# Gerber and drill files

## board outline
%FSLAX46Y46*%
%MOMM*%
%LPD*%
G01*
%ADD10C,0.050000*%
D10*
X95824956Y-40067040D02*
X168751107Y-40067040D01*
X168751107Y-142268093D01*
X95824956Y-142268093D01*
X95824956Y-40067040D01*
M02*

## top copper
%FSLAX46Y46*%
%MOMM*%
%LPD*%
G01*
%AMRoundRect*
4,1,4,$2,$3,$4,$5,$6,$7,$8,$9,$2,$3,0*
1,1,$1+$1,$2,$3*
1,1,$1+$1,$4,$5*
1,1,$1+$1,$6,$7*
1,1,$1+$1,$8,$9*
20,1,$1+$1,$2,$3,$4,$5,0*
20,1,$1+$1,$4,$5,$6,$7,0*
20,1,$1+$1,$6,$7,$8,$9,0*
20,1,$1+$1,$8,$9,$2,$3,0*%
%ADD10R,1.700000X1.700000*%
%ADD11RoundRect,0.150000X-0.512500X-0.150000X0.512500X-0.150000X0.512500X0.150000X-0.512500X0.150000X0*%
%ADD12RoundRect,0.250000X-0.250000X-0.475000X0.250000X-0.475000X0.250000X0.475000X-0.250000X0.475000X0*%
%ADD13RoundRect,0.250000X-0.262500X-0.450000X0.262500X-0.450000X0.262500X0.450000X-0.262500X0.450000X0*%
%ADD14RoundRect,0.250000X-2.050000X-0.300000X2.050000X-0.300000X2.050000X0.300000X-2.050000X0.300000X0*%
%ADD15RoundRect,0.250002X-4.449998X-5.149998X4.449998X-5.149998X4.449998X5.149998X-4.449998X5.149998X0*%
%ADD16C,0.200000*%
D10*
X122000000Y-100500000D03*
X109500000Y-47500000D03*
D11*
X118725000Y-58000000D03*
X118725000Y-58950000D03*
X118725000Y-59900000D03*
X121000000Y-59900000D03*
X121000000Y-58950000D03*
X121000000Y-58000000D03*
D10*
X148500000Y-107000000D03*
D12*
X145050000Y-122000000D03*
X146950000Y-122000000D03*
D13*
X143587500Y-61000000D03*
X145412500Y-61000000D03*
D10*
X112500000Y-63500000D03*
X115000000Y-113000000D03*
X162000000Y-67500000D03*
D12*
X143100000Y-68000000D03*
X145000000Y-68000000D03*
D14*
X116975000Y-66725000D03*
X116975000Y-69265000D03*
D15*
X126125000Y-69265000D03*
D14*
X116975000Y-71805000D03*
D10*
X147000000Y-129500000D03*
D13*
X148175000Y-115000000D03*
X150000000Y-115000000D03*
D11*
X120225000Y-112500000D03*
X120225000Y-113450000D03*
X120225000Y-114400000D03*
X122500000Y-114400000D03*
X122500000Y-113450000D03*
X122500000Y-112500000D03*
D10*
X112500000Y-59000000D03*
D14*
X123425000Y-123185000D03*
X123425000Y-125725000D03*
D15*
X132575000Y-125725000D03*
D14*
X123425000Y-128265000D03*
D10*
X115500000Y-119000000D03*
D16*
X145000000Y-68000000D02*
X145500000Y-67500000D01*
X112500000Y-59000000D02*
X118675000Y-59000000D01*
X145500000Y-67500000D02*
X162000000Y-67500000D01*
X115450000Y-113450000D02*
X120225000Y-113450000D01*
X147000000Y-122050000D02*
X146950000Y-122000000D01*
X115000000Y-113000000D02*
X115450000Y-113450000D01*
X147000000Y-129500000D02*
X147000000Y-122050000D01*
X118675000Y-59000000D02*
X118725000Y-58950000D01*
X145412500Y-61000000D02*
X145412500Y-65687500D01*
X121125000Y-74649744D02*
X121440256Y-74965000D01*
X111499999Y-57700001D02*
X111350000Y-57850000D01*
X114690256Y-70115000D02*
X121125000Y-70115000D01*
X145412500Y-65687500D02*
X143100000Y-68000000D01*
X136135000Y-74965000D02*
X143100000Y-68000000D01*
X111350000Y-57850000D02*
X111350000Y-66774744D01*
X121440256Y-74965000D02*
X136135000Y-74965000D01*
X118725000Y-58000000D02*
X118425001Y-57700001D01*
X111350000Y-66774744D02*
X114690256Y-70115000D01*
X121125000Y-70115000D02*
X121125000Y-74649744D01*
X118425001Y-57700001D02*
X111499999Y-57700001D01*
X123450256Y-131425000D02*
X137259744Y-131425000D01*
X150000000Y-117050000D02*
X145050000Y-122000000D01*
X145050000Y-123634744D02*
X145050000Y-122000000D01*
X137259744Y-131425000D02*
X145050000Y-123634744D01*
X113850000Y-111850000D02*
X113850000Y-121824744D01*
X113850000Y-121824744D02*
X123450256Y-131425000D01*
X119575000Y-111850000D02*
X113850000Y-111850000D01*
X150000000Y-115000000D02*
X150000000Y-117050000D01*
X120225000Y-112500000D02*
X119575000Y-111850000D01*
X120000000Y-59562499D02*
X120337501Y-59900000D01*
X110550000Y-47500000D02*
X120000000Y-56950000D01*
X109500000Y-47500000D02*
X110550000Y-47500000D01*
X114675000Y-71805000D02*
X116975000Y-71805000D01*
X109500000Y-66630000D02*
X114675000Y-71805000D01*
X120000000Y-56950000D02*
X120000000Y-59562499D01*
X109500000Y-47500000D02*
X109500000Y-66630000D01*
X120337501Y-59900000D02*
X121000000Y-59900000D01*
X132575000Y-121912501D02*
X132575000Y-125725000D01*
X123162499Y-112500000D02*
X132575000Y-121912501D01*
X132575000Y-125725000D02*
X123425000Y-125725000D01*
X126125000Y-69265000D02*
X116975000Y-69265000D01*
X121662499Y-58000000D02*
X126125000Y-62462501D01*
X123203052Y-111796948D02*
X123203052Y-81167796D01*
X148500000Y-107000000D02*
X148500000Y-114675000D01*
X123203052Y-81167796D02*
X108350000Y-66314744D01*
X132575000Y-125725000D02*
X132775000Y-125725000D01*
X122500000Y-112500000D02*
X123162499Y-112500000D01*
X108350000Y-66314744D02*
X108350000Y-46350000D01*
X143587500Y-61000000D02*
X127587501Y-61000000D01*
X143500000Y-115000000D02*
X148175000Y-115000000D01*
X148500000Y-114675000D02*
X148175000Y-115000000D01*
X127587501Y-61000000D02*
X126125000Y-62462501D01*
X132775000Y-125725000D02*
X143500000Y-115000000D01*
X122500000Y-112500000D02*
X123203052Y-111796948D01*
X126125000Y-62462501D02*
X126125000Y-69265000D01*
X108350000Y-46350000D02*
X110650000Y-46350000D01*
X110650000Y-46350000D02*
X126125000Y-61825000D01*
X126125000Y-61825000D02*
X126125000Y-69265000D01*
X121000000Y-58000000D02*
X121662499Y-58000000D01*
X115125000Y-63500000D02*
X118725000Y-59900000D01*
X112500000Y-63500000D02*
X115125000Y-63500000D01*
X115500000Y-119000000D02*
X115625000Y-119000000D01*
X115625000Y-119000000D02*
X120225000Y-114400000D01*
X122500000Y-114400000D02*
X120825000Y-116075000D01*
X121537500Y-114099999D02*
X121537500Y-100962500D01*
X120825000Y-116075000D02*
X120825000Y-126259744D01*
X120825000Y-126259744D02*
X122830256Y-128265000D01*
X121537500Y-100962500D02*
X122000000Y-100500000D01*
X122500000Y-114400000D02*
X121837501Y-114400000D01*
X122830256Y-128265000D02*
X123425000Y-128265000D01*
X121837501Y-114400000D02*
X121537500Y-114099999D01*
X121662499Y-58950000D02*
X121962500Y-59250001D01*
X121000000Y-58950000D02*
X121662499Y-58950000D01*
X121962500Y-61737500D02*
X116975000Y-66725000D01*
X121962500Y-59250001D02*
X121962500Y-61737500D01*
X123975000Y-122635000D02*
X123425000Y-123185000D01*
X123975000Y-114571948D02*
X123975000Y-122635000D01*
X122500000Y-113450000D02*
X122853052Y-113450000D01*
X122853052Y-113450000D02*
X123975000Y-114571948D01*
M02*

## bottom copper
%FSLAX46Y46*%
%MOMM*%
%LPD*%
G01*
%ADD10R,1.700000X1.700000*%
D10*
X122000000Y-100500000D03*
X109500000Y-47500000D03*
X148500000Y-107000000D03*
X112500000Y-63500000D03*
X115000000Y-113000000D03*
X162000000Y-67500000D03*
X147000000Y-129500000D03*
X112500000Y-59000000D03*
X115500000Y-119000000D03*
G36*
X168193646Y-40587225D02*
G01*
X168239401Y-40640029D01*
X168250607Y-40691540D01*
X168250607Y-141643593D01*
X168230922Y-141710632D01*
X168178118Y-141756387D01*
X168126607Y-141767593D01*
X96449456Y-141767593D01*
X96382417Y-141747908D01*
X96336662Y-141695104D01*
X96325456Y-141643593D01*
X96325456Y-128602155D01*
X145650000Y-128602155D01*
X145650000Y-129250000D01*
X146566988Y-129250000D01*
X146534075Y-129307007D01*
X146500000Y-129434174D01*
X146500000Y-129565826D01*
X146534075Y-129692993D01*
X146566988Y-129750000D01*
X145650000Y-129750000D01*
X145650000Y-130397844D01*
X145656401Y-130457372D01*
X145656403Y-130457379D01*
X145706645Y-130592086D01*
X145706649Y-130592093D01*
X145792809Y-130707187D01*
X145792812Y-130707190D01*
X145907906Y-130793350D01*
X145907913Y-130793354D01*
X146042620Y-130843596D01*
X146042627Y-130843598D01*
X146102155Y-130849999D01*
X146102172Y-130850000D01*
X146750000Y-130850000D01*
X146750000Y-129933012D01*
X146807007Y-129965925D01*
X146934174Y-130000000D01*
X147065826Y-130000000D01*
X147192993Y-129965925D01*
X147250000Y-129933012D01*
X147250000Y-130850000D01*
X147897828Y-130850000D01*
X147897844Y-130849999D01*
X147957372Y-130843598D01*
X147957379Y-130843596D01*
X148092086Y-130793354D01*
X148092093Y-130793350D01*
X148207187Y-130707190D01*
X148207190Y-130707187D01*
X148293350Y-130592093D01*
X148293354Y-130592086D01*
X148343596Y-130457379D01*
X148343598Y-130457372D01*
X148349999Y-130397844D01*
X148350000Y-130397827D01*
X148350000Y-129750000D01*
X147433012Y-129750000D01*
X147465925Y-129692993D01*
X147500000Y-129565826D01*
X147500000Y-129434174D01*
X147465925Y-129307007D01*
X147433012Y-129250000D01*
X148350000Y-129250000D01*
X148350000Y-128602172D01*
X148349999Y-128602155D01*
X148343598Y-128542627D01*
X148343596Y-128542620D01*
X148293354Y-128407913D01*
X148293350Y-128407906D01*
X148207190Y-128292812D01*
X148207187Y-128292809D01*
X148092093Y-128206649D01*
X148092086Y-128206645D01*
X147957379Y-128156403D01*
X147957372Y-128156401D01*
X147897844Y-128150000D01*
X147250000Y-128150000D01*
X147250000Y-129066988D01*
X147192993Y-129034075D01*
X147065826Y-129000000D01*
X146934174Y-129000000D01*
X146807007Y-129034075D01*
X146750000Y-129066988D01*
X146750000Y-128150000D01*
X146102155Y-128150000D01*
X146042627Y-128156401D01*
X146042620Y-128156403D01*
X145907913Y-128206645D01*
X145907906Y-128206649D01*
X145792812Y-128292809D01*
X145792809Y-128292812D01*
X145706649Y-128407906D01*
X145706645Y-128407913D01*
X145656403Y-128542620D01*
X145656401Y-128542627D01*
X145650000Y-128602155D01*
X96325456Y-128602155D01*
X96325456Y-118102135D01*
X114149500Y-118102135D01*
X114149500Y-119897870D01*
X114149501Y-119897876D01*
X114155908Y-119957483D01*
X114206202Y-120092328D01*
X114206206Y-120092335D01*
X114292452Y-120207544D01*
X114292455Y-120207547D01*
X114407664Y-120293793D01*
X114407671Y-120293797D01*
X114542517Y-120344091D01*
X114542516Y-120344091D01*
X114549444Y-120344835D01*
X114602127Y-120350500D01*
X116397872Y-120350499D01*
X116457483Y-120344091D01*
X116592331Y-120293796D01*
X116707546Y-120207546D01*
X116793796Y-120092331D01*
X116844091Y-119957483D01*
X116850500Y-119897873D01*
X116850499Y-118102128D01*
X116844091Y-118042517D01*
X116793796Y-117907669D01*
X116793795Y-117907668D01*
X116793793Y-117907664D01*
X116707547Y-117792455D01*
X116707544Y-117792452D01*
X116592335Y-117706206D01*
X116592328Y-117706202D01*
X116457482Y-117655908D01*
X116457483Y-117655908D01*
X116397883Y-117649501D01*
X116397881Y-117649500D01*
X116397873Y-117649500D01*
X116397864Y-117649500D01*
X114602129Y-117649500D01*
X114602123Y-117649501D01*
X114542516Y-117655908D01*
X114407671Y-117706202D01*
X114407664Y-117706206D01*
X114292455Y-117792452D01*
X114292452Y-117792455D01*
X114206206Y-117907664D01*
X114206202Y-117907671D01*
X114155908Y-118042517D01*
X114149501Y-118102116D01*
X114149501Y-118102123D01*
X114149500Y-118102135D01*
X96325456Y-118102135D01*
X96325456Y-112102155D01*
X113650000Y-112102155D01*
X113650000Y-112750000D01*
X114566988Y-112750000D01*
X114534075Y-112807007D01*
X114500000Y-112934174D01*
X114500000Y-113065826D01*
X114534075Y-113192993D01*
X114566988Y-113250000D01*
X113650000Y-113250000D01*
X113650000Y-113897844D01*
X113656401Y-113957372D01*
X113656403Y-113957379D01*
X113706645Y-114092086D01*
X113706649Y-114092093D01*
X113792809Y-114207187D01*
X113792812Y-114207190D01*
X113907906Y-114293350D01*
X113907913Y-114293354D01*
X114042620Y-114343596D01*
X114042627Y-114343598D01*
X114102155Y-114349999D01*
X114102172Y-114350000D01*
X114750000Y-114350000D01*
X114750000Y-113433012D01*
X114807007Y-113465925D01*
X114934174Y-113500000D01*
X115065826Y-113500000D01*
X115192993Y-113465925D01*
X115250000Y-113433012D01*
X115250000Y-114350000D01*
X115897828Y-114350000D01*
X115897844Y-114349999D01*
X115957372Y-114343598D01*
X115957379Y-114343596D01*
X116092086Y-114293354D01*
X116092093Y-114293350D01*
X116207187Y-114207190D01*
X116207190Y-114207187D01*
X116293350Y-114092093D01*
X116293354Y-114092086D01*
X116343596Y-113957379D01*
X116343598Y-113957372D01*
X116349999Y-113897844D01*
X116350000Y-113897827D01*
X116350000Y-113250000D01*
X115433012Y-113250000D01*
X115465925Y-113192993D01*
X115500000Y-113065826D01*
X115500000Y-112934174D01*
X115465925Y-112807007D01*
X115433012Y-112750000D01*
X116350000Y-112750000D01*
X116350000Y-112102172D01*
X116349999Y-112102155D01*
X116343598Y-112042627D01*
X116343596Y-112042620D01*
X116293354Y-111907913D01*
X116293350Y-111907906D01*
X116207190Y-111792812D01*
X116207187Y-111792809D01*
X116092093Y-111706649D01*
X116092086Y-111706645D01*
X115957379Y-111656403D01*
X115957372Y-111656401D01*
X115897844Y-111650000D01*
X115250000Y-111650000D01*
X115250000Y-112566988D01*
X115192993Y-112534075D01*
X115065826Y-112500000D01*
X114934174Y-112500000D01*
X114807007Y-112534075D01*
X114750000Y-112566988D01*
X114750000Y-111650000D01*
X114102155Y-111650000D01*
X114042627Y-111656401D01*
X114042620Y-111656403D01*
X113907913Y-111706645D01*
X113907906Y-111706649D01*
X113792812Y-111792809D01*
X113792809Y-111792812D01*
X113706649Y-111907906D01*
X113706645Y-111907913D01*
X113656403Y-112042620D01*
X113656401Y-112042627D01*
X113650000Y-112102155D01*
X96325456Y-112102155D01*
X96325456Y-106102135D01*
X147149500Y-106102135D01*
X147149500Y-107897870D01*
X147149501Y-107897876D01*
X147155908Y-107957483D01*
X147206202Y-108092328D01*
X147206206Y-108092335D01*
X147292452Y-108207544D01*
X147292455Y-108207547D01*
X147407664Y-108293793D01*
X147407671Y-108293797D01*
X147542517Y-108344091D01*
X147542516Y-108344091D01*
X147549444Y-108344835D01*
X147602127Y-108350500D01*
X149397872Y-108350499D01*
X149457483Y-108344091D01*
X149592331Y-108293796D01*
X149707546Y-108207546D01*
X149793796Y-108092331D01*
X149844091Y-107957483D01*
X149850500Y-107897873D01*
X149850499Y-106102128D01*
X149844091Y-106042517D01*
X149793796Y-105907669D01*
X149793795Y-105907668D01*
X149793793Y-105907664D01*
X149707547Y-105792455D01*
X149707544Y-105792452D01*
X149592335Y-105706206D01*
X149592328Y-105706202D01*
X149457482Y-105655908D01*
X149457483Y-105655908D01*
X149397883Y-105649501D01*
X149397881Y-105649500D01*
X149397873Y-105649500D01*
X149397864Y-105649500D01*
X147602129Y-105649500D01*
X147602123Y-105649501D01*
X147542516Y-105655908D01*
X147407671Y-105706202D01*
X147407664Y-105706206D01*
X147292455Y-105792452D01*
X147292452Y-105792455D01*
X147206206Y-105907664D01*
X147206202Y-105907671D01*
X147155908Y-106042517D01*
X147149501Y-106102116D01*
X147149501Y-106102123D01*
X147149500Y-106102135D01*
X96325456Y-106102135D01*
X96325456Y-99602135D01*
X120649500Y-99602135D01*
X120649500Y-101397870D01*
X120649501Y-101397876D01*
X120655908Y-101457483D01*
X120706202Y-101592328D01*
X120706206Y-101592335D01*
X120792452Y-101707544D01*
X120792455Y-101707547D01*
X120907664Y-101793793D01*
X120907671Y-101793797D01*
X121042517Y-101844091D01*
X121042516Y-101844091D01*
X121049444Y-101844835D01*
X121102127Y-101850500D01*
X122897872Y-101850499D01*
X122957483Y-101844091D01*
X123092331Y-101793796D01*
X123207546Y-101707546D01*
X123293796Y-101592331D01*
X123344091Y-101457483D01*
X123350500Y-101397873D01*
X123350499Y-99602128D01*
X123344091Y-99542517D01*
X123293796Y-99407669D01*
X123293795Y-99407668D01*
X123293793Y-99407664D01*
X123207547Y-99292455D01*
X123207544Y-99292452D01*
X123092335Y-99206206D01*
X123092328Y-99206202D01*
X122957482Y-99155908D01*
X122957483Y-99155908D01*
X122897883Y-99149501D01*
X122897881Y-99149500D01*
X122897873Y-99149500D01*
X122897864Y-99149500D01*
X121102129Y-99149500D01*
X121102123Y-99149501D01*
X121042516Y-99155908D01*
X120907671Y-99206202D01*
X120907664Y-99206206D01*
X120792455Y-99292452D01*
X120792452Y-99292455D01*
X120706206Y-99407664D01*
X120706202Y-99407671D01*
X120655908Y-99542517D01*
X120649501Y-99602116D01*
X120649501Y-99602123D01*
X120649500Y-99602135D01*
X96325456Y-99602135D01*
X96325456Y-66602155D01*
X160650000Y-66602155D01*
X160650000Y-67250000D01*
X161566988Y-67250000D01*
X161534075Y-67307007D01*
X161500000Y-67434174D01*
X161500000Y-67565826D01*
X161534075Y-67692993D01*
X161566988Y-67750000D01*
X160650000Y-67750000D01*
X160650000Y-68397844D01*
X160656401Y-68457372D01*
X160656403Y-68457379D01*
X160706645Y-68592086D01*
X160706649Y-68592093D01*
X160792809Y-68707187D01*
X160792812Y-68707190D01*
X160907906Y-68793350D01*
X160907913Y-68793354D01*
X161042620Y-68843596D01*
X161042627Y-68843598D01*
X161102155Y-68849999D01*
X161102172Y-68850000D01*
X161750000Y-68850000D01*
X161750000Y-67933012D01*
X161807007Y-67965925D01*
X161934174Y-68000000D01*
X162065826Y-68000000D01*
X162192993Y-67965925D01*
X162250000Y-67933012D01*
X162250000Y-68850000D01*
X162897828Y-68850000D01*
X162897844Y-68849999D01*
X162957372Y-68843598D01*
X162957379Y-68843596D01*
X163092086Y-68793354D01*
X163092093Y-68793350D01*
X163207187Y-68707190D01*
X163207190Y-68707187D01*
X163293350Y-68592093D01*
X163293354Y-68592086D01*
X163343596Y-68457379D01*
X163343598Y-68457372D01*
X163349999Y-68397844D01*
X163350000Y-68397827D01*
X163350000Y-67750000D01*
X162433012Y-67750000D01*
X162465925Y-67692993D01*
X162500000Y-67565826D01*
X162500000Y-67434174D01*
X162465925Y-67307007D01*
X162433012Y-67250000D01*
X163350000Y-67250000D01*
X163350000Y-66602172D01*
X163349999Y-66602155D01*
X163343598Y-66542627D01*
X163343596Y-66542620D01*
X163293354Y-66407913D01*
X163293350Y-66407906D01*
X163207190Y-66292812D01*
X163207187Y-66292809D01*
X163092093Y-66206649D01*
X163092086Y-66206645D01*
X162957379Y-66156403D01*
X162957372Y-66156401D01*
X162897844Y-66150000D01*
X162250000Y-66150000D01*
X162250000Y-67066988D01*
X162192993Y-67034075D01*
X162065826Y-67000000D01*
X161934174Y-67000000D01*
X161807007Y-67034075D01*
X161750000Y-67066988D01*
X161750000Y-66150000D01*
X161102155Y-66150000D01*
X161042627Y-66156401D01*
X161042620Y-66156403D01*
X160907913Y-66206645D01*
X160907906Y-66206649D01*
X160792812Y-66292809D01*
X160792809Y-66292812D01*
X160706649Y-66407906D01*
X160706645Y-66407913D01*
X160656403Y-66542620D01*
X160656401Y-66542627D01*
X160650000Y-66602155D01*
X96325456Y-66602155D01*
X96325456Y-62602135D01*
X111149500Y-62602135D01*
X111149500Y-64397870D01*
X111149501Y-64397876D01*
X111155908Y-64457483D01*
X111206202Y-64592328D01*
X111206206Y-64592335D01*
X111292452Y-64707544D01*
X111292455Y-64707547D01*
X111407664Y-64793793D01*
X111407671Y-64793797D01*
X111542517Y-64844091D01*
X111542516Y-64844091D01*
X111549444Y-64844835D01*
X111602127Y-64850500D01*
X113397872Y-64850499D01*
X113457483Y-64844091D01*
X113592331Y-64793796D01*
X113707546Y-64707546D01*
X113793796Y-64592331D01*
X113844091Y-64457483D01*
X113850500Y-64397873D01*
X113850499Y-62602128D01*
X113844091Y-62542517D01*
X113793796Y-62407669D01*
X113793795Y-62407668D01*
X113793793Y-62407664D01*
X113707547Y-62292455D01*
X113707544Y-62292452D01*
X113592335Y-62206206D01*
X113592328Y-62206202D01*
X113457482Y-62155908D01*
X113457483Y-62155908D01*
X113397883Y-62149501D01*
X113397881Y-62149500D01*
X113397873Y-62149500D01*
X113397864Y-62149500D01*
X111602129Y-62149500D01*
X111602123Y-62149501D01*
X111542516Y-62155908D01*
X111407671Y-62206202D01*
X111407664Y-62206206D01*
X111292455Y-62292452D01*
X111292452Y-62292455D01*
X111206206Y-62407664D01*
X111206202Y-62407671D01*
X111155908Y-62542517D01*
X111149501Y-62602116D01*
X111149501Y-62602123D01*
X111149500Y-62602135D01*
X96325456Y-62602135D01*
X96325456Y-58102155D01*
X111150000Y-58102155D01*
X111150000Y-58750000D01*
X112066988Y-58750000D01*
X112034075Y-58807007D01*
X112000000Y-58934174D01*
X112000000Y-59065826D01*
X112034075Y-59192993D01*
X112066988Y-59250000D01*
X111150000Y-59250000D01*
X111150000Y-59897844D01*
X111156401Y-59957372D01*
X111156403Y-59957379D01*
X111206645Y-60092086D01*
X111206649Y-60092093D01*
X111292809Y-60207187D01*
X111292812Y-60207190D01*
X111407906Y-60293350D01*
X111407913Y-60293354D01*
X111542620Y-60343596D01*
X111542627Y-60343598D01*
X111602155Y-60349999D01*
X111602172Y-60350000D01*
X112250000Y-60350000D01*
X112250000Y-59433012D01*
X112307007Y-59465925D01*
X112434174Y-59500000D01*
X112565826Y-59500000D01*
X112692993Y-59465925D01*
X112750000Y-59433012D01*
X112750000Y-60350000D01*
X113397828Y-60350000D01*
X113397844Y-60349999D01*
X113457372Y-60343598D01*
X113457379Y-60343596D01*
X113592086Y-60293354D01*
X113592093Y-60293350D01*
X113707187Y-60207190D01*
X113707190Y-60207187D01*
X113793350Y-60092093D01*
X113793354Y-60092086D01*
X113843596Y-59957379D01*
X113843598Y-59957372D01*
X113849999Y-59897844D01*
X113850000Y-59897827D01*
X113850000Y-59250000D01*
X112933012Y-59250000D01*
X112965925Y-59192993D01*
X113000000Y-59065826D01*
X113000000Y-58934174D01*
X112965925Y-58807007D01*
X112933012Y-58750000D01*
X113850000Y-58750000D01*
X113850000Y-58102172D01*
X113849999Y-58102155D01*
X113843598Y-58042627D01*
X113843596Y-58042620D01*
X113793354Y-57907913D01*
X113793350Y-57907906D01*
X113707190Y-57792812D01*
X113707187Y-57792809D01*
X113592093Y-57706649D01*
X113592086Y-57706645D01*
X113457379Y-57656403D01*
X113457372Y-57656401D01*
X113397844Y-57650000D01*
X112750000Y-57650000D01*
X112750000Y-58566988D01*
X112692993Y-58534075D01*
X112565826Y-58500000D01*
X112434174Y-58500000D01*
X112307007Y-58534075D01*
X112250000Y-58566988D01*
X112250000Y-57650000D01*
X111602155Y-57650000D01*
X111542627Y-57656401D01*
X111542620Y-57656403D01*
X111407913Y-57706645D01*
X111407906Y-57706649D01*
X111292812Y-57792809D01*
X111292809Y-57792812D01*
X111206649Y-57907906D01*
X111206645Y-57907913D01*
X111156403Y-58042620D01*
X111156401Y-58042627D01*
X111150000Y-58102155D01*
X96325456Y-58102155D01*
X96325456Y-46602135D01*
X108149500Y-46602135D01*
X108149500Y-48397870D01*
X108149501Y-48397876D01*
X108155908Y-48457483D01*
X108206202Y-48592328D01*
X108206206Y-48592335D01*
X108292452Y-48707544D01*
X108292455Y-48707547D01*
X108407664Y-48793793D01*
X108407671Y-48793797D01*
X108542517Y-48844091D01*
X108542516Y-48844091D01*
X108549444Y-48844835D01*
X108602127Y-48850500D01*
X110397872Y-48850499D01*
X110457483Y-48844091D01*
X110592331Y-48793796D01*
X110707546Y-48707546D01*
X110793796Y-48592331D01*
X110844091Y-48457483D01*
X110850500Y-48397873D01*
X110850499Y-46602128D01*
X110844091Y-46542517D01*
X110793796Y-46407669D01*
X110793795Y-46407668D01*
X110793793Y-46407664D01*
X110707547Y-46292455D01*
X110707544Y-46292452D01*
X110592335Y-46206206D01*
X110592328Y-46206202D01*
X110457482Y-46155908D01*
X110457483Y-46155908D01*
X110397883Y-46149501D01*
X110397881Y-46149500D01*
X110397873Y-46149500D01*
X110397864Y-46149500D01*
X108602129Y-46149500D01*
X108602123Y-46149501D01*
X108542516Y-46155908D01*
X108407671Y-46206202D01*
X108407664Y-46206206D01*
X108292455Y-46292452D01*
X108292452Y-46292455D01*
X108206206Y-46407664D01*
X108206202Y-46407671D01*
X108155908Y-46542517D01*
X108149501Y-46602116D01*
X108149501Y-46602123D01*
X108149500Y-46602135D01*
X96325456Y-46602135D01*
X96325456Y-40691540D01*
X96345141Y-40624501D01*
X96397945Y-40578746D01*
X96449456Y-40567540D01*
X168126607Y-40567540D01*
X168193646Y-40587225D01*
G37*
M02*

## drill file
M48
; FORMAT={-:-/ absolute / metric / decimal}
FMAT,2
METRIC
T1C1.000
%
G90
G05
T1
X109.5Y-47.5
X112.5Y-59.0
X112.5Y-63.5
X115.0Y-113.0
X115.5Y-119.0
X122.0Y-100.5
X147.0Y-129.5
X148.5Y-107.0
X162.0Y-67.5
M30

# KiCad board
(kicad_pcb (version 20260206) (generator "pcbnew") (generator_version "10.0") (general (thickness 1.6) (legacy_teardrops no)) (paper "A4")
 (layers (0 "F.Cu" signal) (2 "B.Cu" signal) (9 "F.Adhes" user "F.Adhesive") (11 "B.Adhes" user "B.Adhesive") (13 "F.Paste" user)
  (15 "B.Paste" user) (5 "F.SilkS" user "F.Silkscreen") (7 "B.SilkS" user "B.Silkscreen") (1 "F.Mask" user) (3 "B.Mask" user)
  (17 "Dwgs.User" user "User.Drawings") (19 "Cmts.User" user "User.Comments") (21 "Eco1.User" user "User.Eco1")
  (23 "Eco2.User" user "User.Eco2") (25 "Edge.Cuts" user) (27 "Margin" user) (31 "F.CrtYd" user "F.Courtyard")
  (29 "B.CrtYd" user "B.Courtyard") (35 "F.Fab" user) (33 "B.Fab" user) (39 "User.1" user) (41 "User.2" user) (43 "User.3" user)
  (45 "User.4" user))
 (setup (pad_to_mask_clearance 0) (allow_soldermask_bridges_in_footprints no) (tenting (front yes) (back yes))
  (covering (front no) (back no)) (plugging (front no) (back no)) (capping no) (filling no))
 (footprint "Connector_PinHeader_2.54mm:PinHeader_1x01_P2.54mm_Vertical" (layer "F.Cu") (at 122 100.5)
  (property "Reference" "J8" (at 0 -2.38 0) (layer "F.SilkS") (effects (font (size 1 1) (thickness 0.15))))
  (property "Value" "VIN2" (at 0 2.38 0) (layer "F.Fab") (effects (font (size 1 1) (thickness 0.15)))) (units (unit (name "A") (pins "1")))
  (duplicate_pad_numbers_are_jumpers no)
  (pad "1" thru_hole rect (at 0 0) (size 1.7 1.7) (drill 1) (layers "*.Cu" "*.Mask") (remove_unused_layers no) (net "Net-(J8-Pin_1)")))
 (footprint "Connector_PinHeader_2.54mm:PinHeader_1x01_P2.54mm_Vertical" (layer "F.Cu") (at 109.5 47.5)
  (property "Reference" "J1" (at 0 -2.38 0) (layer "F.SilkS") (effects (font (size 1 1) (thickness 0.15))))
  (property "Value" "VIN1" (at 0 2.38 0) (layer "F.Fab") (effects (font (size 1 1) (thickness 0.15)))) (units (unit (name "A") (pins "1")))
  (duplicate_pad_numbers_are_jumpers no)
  (pad "1" thru_hole rect (at 0 0) (size 1.7 1.7) (drill 1) (layers "*.Cu" "*.Mask") (remove_unused_layers no) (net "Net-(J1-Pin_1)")))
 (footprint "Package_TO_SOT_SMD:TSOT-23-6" (layer "F.Cu") (at 119.8625 58.95)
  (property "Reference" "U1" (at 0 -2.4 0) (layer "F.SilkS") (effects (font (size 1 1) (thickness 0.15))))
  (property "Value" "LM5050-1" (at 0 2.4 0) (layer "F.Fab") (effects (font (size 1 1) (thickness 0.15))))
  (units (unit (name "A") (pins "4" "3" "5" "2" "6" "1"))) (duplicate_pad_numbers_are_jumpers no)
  (pad "1" smd roundrect (at -1.1375 -0.95) (size 1.325 0.6) (layers "F.Cu" "F.Mask" "F.Paste") (roundrect_rratio 0.25) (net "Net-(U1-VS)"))
  (pad "2" smd roundrect (at -1.1375 0) (size 1.325 0.6) (layers "F.Cu" "F.Mask" "F.Paste") (roundrect_rratio 0.25) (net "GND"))
  (pad "3" smd roundrect (at -1.1375 0.95) (size 1.325 0.6) (layers "F.Cu" "F.Mask" "F.Paste") (roundrect_rratio 0.25)
   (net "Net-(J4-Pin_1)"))
  (pad "4" smd roundrect (at 1.1375 0.95) (size 1.325 0.6) (layers "F.Cu" "F.Mask" "F.Paste") (roundrect_rratio 0.25) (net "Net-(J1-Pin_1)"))
  (pad "5" smd roundrect (at 1.1375 0) (size 1.325 0.6) (layers "F.Cu" "F.Mask" "F.Paste") (roundrect_rratio 0.25) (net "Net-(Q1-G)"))
  (pad "6" smd roundrect (at 1.1375 -0.95) (size 1.325 0.6) (layers "F.Cu" "F.Mask" "F.Paste") (roundrect_rratio 0.25)
   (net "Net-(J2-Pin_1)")))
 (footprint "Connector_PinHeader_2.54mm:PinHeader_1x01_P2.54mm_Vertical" (layer "F.Cu") (at 148.5 107)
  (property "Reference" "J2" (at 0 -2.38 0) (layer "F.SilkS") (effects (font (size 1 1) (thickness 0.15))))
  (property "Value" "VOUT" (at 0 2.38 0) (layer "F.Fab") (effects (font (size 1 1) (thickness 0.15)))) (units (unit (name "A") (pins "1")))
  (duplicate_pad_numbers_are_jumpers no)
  (pad "1" thru_hole rect (at 0 0) (size 1.7 1.7) (drill 1) (layers "*.Cu" "*.Mask") (remove_unused_layers no) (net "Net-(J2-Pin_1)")))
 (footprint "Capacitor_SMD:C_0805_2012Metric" (layer "F.Cu") (at 146 122)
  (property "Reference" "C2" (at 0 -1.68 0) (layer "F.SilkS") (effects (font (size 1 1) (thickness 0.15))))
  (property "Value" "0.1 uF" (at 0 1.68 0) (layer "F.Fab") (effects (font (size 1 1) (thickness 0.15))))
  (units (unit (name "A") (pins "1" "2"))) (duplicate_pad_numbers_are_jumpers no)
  (pad "1" smd roundrect (at -0.95 0) (size 1 1.45) (layers "F.Cu" "F.Mask" "F.Paste") (roundrect_rratio 0.25) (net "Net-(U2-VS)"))
  (pad "2" smd roundrect (at 0.95 0) (size 1 1.45) (layers "F.Cu" "F.Mask" "F.Paste") (roundrect_rratio 0.25) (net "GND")))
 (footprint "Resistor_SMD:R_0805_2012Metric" (layer "F.Cu") (at 144.5 61)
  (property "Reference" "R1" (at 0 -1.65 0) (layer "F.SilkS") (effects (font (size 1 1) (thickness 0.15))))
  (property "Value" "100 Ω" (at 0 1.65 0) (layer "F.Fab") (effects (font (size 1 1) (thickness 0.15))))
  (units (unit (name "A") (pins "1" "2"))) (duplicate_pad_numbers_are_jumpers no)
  (pad "1" smd roundrect (at -0.9125 0) (size 1.025 1.4) (layers "F.Cu" "F.Mask" "F.Paste") (roundrect_rratio 0.243902)
   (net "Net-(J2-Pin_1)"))
  (pad "2" smd roundrect (at 0.9125 0) (size 1.025 1.4) (layers "F.Cu" "F.Mask" "F.Paste") (roundrect_rratio 0.243902) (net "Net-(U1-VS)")))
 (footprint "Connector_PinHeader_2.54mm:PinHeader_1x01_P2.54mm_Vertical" (layer "F.Cu") (at 112.5 63.5)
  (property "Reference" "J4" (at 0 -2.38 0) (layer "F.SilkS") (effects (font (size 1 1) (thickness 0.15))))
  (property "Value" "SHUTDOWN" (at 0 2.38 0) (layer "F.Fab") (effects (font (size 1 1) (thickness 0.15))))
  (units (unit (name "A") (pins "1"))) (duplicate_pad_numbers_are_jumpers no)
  (pad "1" thru_hole rect (at 0 0) (size 1.7 1.7) (drill 1) (layers "*.Cu" "*.Mask") (remove_unused_layers no) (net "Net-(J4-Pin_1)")))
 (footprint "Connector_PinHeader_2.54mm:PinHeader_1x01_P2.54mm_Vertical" (layer "F.Cu") (at 115 113)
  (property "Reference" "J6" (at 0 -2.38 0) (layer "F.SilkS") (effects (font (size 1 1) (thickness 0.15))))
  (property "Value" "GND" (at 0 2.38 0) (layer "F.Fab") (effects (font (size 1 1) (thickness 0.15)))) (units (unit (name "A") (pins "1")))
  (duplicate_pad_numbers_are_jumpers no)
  (pad "1" thru_hole rect (at 0 0) (size 1.7 1.7) (drill 1) (layers "*.Cu" "*.Mask") (remove_unused_layers no) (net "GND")))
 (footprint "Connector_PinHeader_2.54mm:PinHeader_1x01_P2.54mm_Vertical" (layer "F.Cu") (at 162 67.5)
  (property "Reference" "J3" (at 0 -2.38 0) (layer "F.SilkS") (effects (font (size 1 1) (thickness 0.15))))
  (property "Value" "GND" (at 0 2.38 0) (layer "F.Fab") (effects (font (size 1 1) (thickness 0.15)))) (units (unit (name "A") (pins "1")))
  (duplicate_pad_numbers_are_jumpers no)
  (pad "1" thru_hole rect (at 0 0) (size 1.7 1.7) (drill 1) (layers "*.Cu" "*.Mask") (remove_unused_layers no) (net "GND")))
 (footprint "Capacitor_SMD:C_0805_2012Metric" (layer "F.Cu") (at 144.05 68)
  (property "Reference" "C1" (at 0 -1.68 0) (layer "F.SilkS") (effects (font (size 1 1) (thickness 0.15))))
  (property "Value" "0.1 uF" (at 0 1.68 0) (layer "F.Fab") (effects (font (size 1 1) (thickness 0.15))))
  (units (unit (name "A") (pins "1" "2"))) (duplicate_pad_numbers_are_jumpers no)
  (pad "1" smd roundrect (at -0.95 0) (size 1 1.45) (layers "F.Cu" "F.Mask" "F.Paste") (roundrect_rratio 0.25) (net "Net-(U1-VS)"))
  (pad "2" smd roundrect (at 0.95 0) (size 1 1.45) (layers "F.Cu" "F.Mask" "F.Paste") (roundrect_rratio 0.25) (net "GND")))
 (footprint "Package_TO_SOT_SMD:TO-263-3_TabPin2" (layer "F.Cu") (at 124.625 69.265)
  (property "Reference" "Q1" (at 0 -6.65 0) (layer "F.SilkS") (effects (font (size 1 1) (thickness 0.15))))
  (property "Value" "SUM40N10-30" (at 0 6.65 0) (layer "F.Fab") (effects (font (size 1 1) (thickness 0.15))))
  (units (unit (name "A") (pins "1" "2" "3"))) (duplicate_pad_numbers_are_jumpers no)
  (pad "" smd roundrect (at -0.925 -2.775) (size 4.55 5.25) (layers "F.Paste") (roundrect_rratio 0.054945))
  (pad "" smd roundrect (at -0.925 2.775) (size 4.55 5.25) (layers "F.Paste") (roundrect_rratio 0.054945))
  (pad "" smd roundrect (at 3.925 -2.775) (size 4.55 5.25) (layers "F.Paste") (roundrect_rratio 0.054945))
  (pad "" smd roundrect (at 3.925 2.775) (size 4.55 5.25) (layers "F.Paste") (roundrect_rratio 0.054945))
  (pad "1" smd roundrect (at -7.65 -2.54) (size 4.6 1.1) (layers "F.Cu" "F.Mask" "F.Paste") (roundrect_rratio 0.227273) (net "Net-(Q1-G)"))
  (pad "2" smd roundrect (at -7.65 0) (size 4.6 1.1) (layers "F.Cu" "F.Mask" "F.Paste") (roundrect_rratio 0.227273) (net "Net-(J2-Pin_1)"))
  (pad "2" smd roundrect (at 1.5 0) (size 9.4 10.8) (layers "F.Cu" "F.Mask") (roundrect_rratio 0.026596) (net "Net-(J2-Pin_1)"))
  (pad "3" smd roundrect (at -7.65 2.54) (size 4.6 1.1) (layers "F.Cu" "F.Mask" "F.Paste") (roundrect_rratio 0.227273)
   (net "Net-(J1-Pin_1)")))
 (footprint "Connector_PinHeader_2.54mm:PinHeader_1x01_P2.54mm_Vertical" (layer "F.Cu") (at 147 129.5)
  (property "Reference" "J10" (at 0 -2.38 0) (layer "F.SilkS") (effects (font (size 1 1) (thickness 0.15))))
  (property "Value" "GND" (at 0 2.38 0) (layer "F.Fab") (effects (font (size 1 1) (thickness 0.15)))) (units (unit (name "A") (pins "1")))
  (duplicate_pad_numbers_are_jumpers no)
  (pad "1" thru_hole rect (at 0 0) (size 1.7 1.7) (drill 1) (layers "*.Cu" "*.Mask") (remove_unused_layers no) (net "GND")))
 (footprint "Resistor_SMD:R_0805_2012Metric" (layer "F.Cu") (at 149.0875 115)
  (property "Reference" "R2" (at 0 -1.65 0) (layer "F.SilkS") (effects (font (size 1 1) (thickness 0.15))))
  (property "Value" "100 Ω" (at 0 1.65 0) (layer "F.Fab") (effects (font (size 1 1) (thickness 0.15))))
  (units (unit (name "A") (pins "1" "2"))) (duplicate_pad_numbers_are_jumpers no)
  (pad "1" smd roundrect (at -0.9125 0) (size 1.025 1.4) (layers "F.Cu" "F.Mask" "F.Paste") (roundrect_rratio 0.243902)
   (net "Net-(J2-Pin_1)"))
  (pad "2" smd roundrect (at 0.9125 0) (size 1.025 1.4) (layers "F.Cu" "F.Mask" "F.Paste") (roundrect_rratio 0.243902) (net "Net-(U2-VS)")))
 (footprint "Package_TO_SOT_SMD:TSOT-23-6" (layer "F.Cu") (at 121.3625 113.45)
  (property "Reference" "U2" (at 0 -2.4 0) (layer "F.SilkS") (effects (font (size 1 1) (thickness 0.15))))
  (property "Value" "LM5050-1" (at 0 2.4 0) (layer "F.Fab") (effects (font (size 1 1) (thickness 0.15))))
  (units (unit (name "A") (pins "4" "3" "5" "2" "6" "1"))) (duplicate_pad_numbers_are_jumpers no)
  (pad "1" smd roundrect (at -1.1375 -0.95) (size 1.325 0.6) (layers "F.Cu" "F.Mask" "F.Paste") (roundrect_rratio 0.25) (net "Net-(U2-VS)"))
  (pad "2" smd roundrect (at -1.1375 0) (size 1.325 0.6) (layers "F.Cu" "F.Mask" "F.Paste") (roundrect_rratio 0.25) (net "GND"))
  (pad "3" smd roundrect (at -1.1375 0.95) (size 1.325 0.6) (layers "F.Cu" "F.Mask" "F.Paste") (roundrect_rratio 0.25)
   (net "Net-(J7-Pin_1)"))
  (pad "4" smd roundrect (at 1.1375 0.95) (size 1.325 0.6) (layers "F.Cu" "F.Mask" "F.Paste") (roundrect_rratio 0.25) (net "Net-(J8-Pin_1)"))
  (pad "5" smd roundrect (at 1.1375 0) (size 1.325 0.6) (layers "F.Cu" "F.Mask" "F.Paste") (roundrect_rratio 0.25) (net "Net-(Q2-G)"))
  (pad "6" smd roundrect (at 1.1375 -0.95) (size 1.325 0.6) (layers "F.Cu" "F.Mask" "F.Paste") (roundrect_rratio 0.25)
   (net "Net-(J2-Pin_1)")))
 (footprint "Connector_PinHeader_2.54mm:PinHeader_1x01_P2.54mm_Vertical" (layer "F.Cu") (at 112.5 59)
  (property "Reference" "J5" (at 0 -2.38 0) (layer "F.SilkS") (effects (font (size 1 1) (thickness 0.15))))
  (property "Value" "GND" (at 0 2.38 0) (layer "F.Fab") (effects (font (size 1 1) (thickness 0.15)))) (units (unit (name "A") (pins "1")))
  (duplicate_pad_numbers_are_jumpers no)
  (pad "1" thru_hole rect (at 0 0) (size 1.7 1.7) (drill 1) (layers "*.Cu" "*.Mask") (remove_unused_layers no) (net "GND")))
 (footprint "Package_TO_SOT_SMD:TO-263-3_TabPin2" (layer "F.Cu") (at 131.075 125.725)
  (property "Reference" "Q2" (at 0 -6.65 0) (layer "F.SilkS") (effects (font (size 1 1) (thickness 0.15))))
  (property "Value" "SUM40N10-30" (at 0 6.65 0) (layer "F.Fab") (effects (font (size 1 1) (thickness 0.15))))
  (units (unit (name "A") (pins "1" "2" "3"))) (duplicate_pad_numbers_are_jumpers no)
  (pad "" smd roundrect (at -0.925 -2.775) (size 4.55 5.25) (layers "F.Paste") (roundrect_rratio 0.054945))
  (pad "" smd roundrect (at -0.925 2.775) (size 4.55 5.25) (layers "F.Paste") (roundrect_rratio 0.054945))
  (pad "" smd roundrect (at 3.925 -2.775) (size 4.55 5.25) (layers "F.Paste") (roundrect_rratio 0.054945))
  (pad "" smd roundrect (at 3.925 2.775) (size 4.55 5.25) (layers "F.Paste") (roundrect_rratio 0.054945))
  (pad "1" smd roundrect (at -7.65 -2.54) (size 4.6 1.1) (layers "F.Cu" "F.Mask" "F.Paste") (roundrect_rratio 0.227273) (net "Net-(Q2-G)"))
  (pad "2" smd roundrect (at -7.65 0) (size 4.6 1.1) (layers "F.Cu" "F.Mask" "F.Paste") (roundrect_rratio 0.227273) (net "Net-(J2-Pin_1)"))
  (pad "2" smd roundrect (at 1.5 0) (size 9.4 10.8) (layers "F.Cu" "F.Mask") (roundrect_rratio 0.026596) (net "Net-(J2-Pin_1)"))
  (pad "3" smd roundrect (at -7.65 2.54) (size 4.6 1.1) (layers "F.Cu" "F.Mask" "F.Paste") (roundrect_rratio 0.227273)
   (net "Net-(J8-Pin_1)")))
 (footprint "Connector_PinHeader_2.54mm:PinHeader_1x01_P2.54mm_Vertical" (layer "F.Cu") (at 115.5 119)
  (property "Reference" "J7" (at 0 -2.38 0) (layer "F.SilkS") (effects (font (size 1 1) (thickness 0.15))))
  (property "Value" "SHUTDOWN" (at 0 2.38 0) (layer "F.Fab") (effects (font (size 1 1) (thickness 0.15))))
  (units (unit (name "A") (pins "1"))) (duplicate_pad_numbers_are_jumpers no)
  (pad "1" thru_hole rect (at 0 0) (size 1.7 1.7) (drill 1) (layers "*.Cu" "*.Mask") (remove_unused_layers no) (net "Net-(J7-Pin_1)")))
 (gr_rect (start 95.824956 40.06704) (end 168.751107 142.268093) (stroke (width 0.05) (type default)) (fill no) (layer "Edge.Cuts"))
 (segment (start 145 68) (end 145.5 67.5) (width 0.2) (layer "F.Cu") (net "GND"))
 (segment (start 112.5 59) (end 118.675 59) (width 0.2) (layer "F.Cu") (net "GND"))
 (segment (start 145.5 67.5) (end 162 67.5) (width 0.2) (layer "F.Cu") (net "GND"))
 (segment (start 115.45 113.45) (end 120.225 113.45) (width 0.2) (layer "F.Cu") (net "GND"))
 (segment (start 147 122.05) (end 146.95 122) (width 0.2) (layer "F.Cu") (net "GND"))
 (segment (start 115 113) (end 115.45 113.45) (width 0.2) (layer "F.Cu") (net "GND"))
 (segment (start 147 129.5) (end 147 122.05) (width 0.2) (layer "F.Cu") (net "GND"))
 (segment (start 118.675 59) (end 118.725 58.95) (width 0.2) (layer "F.Cu") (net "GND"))
 (segment (start 145.4125 61) (end 145.4125 65.6875) (width 0.2) (layer "F.Cu") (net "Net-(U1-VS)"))
 (segment (start 121.125 74.649744) (end 121.440256 74.965) (width 0.2) (layer "F.Cu") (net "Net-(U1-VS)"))
 (segment (start 111.499999 57.700001) (end 111.35 57.85) (width 0.2) (layer "F.Cu") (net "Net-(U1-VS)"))
 (segment (start 114.690256 70.115) (end 121.125 70.115) (width 0.2) (layer "F.Cu") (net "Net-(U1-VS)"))
 (segment (start 145.4125 65.6875) (end 143.1 68) (width 0.2) (layer "F.Cu") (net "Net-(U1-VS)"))
 (segment (start 136.135 74.965) (end 143.1 68) (width 0.2) (layer "F.Cu") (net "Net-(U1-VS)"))
 (segment (start 111.35 57.85) (end 111.35 66.774744) (width 0.2) (layer "F.Cu") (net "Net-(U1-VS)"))
 (segment (start 121.440256 74.965) (end 136.135 74.965) (width 0.2) (layer "F.Cu") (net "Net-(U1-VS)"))
 (segment (start 118.725 58) (end 118.425001 57.700001) (width 0.2) (layer "F.Cu") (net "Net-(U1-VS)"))
 (segment (start 111.35 66.774744) (end 114.690256 70.115) (width 0.2) (layer "F.Cu") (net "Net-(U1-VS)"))
 (segment (start 121.125 70.115) (end 121.125 74.649744) (width 0.2) (layer "F.Cu") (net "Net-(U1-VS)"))
 (segment (start 118.425001 57.700001) (end 111.499999 57.700001) (width 0.2) (layer "F.Cu") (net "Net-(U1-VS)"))
 (segment (start 123.450256 131.425) (end 137.259744 131.425) (width 0.2) (layer "F.Cu") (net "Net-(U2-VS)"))
 (segment (start 150 117.05) (end 145.05 122) (width 0.2) (layer "F.Cu") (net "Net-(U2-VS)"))
 (segment (start 145.05 123.634744) (end 145.05 122) (width 0.2) (layer "F.Cu") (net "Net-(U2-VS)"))
 (segment (start 137.259744 131.425) (end 145.05 123.634744) (width 0.2) (layer "F.Cu") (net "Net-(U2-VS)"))
 (segment (start 113.85 111.85) (end 113.85 121.824744) (width 0.2) (layer "F.Cu") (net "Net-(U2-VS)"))
 (segment (start 113.85 121.824744) (end 123.450256 131.425) (width 0.2) (layer "F.Cu") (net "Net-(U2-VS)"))
 (segment (start 119.575 111.85) (end 113.85 111.85) (width 0.2) (layer "F.Cu") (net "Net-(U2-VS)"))
 (segment (start 150 115) (end 150 117.05) (width 0.2) (layer "F.Cu") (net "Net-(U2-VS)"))
 (segment (start 120.225 112.5) (end 119.575 111.85) (width 0.2) (layer "F.Cu") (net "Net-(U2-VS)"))
 (segment (start 120 59.562499) (end 120.337501 59.9) (width 0.2) (layer "F.Cu") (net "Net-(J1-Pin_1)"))
 (segment (start 110.55 47.5) (end 120 56.95) (width 0.2) (layer "F.Cu") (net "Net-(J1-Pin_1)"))
 (segment (start 109.5 47.5) (end 110.55 47.5) (width 0.2) (layer "F.Cu") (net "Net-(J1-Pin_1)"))
 (segment (start 114.675 71.805) (end 116.975 71.805) (width 0.2) (layer "F.Cu") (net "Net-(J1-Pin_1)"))
 (segment (start 109.5 66.63) (end 114.675 71.805) (width 0.2) (layer "F.Cu") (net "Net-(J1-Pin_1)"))
 (segment (start 120 56.95) (end 120 59.562499) (width 0.2) (layer "F.Cu") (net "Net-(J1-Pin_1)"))
 (segment (start 109.5 47.5) (end 109.5 66.63) (width 0.2) (layer "F.Cu") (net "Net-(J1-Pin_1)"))
 (segment (start 120.337501 59.9) (end 121 59.9) (width 0.2) (layer "F.Cu") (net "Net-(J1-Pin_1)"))
 (segment (start 132.575 121.912501) (end 132.575 125.725) (width 0.2) (layer "F.Cu") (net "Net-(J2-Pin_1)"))
 (segment (start 123.162499 112.5) (end 132.575 121.912501) (width 0.2) (layer "F.Cu") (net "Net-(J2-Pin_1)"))
 (segment (start 132.575 125.725) (end 123.425 125.725) (width 0.2) (layer "F.Cu") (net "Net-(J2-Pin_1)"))
 (segment (start 126.125 69.265) (end 116.975 69.265) (width 0.2) (layer "F.Cu") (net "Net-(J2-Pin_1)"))
 (segment (start 121.662499 58) (end 126.125 62.462501) (width 0.2) (layer "F.Cu") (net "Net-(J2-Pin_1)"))
 (segment (start 123.203052 111.796948) (end 123.203052 81.167796) (width 0.2) (layer "F.Cu") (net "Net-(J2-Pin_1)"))
 (segment (start 148.5 107) (end 148.5 114.675) (width 0.2) (layer "F.Cu") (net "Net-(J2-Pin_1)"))
 (segment (start 123.203052 81.167796) (end 108.35 66.314744) (width 0.2) (layer "F.Cu") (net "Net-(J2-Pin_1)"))
 (segment (start 132.575 125.725) (end 132.775 125.725) (width 0.2) (layer "F.Cu") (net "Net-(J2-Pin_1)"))
 (segment (start 122.5 112.5) (end 123.162499 112.5) (width 0.2) (layer "F.Cu") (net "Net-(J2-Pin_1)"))
 (segment (start 108.35 66.314744) (end 108.35 46.35) (width 0.2) (layer "F.Cu") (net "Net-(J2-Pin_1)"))
 (segment (start 143.5875 61) (end 127.587501 61) (width 0.2) (layer "F.Cu") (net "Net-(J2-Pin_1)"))
 (segment (start 143.5 115) (end 148.175 115) (width 0.2) (layer "F.Cu") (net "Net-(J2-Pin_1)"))
 (segment (start 148.5 114.675) (end 148.175 115) (width 0.2) (layer "F.Cu") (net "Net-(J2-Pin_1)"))
 (segment (start 127.587501 61) (end 126.125 62.462501) (width 0.2) (layer "F.Cu") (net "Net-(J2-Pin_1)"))
 (segment (start 132.775 125.725) (end 143.5 115) (width 0.2) (layer "F.Cu") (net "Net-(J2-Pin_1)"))
 (segment (start 122.5 112.5) (end 123.203052 111.796948) (width 0.2) (layer "F.Cu") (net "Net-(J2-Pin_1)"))
 (segment (start 126.125 62.462501) (end 126.125 69.265) (width 0.2) (layer "F.Cu") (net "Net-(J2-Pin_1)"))
 (segment (start 108.35 46.35) (end 110.65 46.35) (width 0.2) (layer "F.Cu") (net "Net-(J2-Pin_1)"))
 (segment (start 110.65 46.35) (end 126.125 61.825) (width 0.2) (layer "F.Cu") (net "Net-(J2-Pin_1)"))
 (segment (start 126.125 61.825) (end 126.125 69.265) (width 0.2) (layer "F.Cu") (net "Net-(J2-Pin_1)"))
 (segment (start 121 58) (end 121.662499 58) (width 0.2) (layer "F.Cu") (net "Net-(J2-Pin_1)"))
 (segment (start 115.125 63.5) (end 118.725 59.9) (width 0.2) (layer "F.Cu") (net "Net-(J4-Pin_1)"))
 (segment (start 112.5 63.5) (end 115.125 63.5) (width 0.2) (layer "F.Cu") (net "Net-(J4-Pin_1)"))
 (segment (start 115.5 119) (end 115.625 119) (width 0.2) (layer "F.Cu") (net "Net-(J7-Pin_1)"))
 (segment (start 115.625 119) (end 120.225 114.4) (width 0.2) (layer "F.Cu") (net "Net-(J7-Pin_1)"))
 (segment (start 122.5 114.4) (end 120.825 116.075) (width 0.2) (layer "F.Cu") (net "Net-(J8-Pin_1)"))
 (segment (start 121.5375 114.099999) (end 121.5375 100.9625) (width 0.2) (layer "F.Cu") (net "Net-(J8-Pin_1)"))
 (segment (start 120.825 116.075) (end 120.825 126.259744) (width 0.2) (layer "F.Cu") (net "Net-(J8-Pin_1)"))
 (segment (start 120.825 126.259744) (end 122.830256 128.265) (width 0.2) (layer "F.Cu") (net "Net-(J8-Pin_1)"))
 (segment (start 121.5375 100.9625) (end 122 100.5) (width 0.2) (layer "F.Cu") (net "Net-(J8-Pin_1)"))
 (segment (start 122.5 114.4) (end 121.837501 114.4) (width 0.2) (layer "F.Cu") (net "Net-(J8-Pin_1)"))
 (segment (start 122.830256 128.265) (end 123.425 128.265) (width 0.2) (layer "F.Cu") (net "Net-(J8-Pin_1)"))
 (segment (start 121.837501 114.4) (end 121.5375 114.099999) (width 0.2) (layer "F.Cu") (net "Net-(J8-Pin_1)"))
 (segment (start 121.662499 58.95) (end 121.9625 59.250001) (width 0.2) (layer "F.Cu") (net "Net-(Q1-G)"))
 (segment (start 121 58.95) (end 121.662499 58.95) (width 0.2) (layer "F.Cu") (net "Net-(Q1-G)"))
 (segment (start 121.9625 61.7375) (end 116.975 66.725) (width 0.2) (layer "F.Cu") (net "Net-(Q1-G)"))
 (segment (start 121.9625 59.250001) (end 121.9625 61.7375) (width 0.2) (layer "F.Cu") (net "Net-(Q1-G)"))
 (segment (start 123.975 122.635) (end 123.425 123.185) (width 0.2) (layer "F.Cu") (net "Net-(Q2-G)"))
 (segment (start 123.975 114.571948) (end 123.975 122.635) (width 0.2) (layer "F.Cu") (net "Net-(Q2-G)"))
 (segment (start 122.5 113.45) (end 122.853052 113.45) (width 0.2) (layer "F.Cu") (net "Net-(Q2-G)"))
 (segment (start 122.853052 113.45) (end 123.975 114.571948) (width 0.2) (layer "F.Cu") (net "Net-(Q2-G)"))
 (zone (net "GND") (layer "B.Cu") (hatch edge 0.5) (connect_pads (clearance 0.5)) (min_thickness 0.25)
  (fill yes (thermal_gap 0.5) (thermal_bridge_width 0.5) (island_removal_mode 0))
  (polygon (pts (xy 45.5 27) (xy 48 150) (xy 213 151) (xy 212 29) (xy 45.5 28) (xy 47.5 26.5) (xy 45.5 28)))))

